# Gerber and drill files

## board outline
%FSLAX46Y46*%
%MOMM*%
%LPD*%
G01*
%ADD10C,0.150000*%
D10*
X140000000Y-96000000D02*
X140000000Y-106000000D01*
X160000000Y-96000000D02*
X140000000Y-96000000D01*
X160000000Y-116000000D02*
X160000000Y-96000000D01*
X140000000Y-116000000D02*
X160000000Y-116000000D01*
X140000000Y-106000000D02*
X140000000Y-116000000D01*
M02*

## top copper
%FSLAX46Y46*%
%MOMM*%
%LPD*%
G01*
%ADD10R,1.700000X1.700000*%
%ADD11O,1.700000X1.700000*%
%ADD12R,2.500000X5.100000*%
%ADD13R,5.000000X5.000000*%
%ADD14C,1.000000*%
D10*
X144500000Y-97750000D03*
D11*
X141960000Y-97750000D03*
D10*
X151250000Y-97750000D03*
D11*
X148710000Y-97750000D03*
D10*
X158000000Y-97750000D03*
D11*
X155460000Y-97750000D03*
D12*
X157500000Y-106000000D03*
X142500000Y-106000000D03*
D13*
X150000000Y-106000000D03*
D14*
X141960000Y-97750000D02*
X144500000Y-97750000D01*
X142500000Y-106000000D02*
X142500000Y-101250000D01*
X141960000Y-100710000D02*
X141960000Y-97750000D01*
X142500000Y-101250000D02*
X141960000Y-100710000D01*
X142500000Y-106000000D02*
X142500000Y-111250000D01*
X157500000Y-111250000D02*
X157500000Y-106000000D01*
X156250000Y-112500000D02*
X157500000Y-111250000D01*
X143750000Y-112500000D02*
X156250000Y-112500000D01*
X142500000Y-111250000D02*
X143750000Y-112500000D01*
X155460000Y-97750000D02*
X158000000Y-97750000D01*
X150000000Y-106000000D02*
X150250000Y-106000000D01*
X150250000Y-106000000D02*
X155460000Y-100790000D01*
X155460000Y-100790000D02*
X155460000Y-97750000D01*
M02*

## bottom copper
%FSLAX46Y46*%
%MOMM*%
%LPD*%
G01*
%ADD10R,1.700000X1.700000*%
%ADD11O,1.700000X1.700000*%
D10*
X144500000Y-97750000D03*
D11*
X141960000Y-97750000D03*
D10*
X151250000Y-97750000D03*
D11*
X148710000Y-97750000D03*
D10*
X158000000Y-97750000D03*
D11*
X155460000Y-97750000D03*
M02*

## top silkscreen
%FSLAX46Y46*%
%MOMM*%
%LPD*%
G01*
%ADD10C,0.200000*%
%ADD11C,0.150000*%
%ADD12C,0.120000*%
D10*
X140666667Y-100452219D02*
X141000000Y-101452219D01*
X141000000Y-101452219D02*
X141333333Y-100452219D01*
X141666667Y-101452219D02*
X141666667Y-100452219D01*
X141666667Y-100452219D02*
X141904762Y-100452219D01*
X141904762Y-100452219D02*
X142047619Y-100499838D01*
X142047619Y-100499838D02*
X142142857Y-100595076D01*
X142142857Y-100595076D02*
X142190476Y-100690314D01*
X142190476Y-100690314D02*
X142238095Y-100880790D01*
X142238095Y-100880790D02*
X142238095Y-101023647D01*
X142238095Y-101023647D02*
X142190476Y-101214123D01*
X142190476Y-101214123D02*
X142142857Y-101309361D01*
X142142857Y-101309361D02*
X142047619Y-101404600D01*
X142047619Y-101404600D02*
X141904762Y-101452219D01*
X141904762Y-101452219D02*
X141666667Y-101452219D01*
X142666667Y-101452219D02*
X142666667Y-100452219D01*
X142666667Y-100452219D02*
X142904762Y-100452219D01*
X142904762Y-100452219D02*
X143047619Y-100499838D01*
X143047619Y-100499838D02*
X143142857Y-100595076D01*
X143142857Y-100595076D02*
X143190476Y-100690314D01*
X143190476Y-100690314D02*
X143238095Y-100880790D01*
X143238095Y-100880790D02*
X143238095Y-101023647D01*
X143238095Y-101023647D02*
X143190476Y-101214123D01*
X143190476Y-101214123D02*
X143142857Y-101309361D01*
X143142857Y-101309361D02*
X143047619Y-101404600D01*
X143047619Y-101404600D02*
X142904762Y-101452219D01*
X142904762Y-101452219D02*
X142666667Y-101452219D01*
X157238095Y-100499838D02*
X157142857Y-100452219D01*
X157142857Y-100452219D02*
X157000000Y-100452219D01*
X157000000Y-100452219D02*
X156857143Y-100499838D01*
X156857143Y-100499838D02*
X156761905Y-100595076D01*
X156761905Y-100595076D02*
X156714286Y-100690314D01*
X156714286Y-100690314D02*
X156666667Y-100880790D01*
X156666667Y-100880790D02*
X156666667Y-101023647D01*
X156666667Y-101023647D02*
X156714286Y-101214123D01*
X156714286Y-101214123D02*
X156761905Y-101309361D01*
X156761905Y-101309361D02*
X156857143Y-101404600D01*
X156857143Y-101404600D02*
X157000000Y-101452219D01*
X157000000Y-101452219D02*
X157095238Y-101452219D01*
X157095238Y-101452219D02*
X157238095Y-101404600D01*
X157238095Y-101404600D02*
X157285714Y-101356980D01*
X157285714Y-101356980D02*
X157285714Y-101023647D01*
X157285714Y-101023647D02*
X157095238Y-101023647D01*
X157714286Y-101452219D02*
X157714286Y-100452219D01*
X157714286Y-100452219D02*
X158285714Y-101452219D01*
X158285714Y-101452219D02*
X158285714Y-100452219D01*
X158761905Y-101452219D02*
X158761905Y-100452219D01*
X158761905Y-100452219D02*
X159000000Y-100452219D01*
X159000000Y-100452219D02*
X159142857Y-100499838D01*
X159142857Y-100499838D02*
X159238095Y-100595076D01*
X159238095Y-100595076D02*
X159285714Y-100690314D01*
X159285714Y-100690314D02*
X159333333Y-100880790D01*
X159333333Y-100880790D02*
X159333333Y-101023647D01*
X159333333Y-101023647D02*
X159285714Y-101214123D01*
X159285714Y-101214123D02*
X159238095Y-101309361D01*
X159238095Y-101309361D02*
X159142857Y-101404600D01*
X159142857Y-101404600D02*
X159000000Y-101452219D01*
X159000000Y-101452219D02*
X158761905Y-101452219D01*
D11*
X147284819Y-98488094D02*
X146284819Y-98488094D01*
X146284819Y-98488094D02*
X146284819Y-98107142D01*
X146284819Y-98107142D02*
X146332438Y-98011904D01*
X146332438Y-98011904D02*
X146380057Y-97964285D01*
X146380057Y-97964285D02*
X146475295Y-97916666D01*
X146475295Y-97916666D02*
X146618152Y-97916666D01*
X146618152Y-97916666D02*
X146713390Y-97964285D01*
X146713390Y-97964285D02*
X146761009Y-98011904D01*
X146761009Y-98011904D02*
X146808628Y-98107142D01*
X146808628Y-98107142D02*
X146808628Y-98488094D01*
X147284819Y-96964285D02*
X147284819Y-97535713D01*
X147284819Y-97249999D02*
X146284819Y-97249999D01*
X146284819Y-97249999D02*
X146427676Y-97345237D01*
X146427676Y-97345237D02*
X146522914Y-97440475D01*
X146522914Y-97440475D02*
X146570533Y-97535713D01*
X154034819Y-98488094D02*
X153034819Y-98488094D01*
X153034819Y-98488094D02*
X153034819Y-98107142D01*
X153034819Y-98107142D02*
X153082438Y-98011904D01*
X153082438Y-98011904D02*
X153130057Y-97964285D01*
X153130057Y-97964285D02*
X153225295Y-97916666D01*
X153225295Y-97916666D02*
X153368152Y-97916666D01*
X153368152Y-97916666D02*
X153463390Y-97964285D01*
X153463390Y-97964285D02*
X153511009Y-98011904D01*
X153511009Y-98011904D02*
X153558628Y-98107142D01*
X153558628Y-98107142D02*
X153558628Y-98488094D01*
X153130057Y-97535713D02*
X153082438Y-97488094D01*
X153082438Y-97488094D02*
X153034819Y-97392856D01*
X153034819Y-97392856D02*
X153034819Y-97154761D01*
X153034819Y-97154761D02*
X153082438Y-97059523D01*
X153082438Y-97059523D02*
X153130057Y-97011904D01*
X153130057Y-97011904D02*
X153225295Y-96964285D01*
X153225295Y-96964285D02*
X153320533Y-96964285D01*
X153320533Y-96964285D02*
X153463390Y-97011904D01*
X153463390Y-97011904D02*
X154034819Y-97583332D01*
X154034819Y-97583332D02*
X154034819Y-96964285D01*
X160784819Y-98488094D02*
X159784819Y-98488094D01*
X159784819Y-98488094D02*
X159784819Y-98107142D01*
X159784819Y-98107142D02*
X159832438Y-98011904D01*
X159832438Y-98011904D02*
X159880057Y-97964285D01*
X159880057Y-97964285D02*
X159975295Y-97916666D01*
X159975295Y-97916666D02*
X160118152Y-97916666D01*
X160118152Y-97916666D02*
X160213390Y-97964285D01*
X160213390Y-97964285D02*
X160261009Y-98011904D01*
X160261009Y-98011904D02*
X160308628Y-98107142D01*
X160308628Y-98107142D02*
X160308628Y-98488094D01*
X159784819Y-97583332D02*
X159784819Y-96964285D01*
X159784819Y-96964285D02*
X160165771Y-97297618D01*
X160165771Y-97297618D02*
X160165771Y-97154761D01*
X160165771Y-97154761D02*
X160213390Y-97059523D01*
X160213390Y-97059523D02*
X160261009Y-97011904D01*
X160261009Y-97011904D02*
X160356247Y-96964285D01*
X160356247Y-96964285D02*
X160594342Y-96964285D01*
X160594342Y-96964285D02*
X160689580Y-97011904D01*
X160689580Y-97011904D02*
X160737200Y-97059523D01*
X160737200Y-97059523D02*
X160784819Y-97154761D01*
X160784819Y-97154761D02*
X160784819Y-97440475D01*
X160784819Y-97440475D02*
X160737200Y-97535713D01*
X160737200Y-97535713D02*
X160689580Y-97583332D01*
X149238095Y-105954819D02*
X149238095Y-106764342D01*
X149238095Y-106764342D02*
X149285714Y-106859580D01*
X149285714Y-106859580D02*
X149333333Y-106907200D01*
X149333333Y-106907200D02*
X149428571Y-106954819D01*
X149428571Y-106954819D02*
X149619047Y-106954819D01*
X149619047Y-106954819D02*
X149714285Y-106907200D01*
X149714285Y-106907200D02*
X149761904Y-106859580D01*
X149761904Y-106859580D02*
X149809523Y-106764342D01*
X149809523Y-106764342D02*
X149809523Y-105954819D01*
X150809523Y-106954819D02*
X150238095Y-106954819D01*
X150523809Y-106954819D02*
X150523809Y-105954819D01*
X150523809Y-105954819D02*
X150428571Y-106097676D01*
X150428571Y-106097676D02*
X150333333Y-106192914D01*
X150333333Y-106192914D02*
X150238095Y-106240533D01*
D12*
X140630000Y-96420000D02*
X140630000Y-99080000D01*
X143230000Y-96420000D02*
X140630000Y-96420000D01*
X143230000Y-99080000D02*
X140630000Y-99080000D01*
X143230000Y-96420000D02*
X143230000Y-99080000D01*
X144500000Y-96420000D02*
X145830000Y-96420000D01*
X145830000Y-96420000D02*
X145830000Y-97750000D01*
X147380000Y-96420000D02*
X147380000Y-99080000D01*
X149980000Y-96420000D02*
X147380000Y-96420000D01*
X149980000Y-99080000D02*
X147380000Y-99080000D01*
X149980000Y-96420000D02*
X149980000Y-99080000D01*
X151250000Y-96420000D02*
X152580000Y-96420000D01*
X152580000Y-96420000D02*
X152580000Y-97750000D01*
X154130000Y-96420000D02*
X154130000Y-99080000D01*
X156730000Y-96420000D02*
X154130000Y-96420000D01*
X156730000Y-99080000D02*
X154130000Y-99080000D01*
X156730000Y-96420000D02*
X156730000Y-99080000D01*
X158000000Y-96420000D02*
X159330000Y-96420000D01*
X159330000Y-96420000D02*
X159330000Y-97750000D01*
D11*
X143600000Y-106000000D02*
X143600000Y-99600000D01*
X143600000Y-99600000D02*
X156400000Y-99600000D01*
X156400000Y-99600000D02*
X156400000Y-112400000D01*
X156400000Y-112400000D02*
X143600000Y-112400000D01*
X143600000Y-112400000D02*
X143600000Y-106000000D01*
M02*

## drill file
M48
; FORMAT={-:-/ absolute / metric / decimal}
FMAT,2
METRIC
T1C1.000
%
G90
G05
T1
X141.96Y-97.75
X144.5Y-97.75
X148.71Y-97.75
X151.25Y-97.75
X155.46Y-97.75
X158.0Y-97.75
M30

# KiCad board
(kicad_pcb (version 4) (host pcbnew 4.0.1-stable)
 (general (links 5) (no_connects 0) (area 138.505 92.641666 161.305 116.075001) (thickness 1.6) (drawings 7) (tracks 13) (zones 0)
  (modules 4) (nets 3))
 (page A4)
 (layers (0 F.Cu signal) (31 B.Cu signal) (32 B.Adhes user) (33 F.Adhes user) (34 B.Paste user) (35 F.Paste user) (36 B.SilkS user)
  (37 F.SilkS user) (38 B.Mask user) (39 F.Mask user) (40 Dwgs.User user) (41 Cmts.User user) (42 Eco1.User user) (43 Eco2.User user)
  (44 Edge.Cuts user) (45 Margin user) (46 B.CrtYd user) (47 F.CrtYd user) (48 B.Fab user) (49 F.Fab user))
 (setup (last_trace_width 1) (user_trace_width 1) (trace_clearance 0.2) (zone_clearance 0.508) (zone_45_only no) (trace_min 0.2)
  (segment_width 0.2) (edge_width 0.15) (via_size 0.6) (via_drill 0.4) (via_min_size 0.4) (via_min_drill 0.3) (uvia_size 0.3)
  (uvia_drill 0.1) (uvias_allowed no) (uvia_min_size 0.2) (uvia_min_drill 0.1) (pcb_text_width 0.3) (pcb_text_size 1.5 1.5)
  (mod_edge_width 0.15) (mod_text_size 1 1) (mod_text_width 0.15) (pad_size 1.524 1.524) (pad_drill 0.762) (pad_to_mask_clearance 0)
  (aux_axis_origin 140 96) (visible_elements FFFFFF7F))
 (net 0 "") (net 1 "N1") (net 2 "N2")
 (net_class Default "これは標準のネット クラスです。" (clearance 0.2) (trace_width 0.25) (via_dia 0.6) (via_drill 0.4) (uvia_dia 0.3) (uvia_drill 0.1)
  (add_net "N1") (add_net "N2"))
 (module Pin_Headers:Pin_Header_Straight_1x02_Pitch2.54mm (layer F.Cu) (at 144.5 97.75 270)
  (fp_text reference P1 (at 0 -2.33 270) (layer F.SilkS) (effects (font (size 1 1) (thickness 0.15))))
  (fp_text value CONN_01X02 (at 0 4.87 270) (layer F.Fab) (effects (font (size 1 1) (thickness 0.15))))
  (fp_line (start -1.33 3.87) (end 1.33 3.87) (layer F.SilkS) (width 0.12))
  (fp_line (start -1.33 1.27) (end -1.33 3.87) (layer F.SilkS) (width 0.12))
  (fp_line (start 1.33 1.27) (end 1.33 3.87) (layer F.SilkS) (width 0.12))
  (fp_line (start -1.33 1.27) (end 1.33 1.27) (layer F.SilkS) (width 0.12))
  (fp_line (start -1.33 0) (end -1.33 -1.33) (layer F.SilkS) (width 0.12))
  (fp_line (start -1.33 -1.33) (end 0 -1.33) (layer F.SilkS) (width 0.12))
  (pad 1 thru_hole rect (at 0 0 270) (size 1.7 1.7) (drill 1) (layers *.Cu *.Mask) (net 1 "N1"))
  (pad 2 thru_hole oval (at 0 2.54 270) (size 1.7 1.7) (drill 1) (layers *.Cu *.Mask) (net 1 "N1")))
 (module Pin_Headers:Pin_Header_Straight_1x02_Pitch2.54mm (layer F.Cu) (at 151.25 97.75 270)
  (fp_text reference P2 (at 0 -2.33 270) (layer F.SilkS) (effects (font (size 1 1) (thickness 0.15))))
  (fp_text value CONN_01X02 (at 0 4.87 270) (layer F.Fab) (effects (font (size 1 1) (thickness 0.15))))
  (fp_line (start -1.33 3.87) (end 1.33 3.87) (layer F.SilkS) (width 0.12))
  (fp_line (start -1.33 1.27) (end -1.33 3.87) (layer F.SilkS) (width 0.12))
  (fp_line (start 1.33 1.27) (end 1.33 3.87) (layer F.SilkS) (width 0.12))
  (fp_line (start -1.33 1.27) (end 1.33 1.27) (layer F.SilkS) (width 0.12))
  (fp_line (start -1.33 0) (end -1.33 -1.33) (layer F.SilkS) (width 0.12))
  (fp_line (start -1.33 -1.33) (end 0 -1.33) (layer F.SilkS) (width 0.12))
  (pad 1 thru_hole rect (at 0 0 270) (size 1.7 1.7) (drill 1) (layers *.Cu *.Mask))
  (pad 2 thru_hole oval (at 0 2.54 270) (size 1.7 1.7) (drill 1) (layers *.Cu *.Mask)))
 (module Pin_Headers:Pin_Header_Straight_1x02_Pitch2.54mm (layer F.Cu) (at 158 97.75 270)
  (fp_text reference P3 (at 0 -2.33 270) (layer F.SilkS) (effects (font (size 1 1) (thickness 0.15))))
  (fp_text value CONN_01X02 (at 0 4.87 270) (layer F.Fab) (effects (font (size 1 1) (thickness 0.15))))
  (fp_line (start -1.33 3.87) (end 1.33 3.87) (layer F.SilkS) (width 0.12))
  (fp_line (start -1.33 1.27) (end -1.33 3.87) (layer F.SilkS) (width 0.12))
  (fp_line (start 1.33 1.27) (end 1.33 3.87) (layer F.SilkS) (width 0.12))
  (fp_line (start -1.33 1.27) (end 1.33 1.27) (layer F.SilkS) (width 0.12))
  (fp_line (start -1.33 0) (end -1.33 -1.33) (layer F.SilkS) (width 0.12))
  (fp_line (start -1.33 -1.33) (end 0 -1.33) (layer F.SilkS) (width 0.12))
  (pad 1 thru_hole rect (at 0 0 270) (size 1.7 1.7) (drill 1) (layers *.Cu *.Mask) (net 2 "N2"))
  (pad 2 thru_hole oval (at 0 2.54 270) (size 1.7 1.7) (drill 1) (layers *.Cu *.Mask) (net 2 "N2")))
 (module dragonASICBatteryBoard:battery (layer F.Cu) (at 150 106)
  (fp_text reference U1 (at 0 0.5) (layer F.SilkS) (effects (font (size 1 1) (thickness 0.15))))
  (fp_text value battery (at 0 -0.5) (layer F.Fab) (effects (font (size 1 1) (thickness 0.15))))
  (fp_line (start -6.4 0) (end -6.4 -6.4) (layer F.SilkS) (width 0.15))
  (fp_line (start -6.4 -6.4) (end 6.4 -6.4) (layer F.SilkS) (width 0.15))
  (fp_line (start 6.4 -6.4) (end 6.4 6.4) (layer F.SilkS) (width 0.15))
  (fp_line (start 6.4 6.4) (end -6.4 6.4) (layer F.SilkS) (width 0.15))
  (fp_line (start -6.4 6.4) (end -6.4 0) (layer F.SilkS) (width 0.15))
  (pad 2 smd rect (at 7.5 0) (size 2.5 5.1) (layers F.Cu F.Paste F.Mask) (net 1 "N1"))
  (pad 2 smd rect (at -7.5 0) (size 2.5 5.1) (layers F.Cu F.Paste F.Mask) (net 1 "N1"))
  (pad 1 smd rect (at 0 0) (size 5 5) (layers F.Cu F.Paste F.Mask) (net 2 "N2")))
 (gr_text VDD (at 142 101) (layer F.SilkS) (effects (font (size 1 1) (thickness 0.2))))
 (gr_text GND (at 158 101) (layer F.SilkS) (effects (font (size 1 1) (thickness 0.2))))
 (gr_line (start 140 96) (end 140 106) (angle 90) (layer Edge.Cuts) (width 0.15))
 (gr_line (start 160 96) (end 140 96) (angle 90) (layer Edge.Cuts) (width 0.15))
 (gr_line (start 160 116) (end 160 96) (angle 90) (layer Edge.Cuts) (width 0.15))
 (gr_line (start 140 116) (end 160 116) (angle 90) (layer Edge.Cuts) (width 0.15))
 (gr_line (start 140 106) (end 140 116) (angle 90) (layer Edge.Cuts) (width 0.15))
 (segment (start 141.96 97.75) (end 144.5 97.75) (width 1) (layer F.Cu) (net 1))
 (segment (start 142.5 106) (end 142.5 101.25) (width 1) (layer F.Cu) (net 1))
 (segment (start 141.96 100.71) (end 141.96 97.75) (width 1) (layer F.Cu) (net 1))
 (segment (start 142.5 101.25) (end 141.96 100.71) (width 1) (layer F.Cu) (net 1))
 (segment (start 142.5 106) (end 142.5 111.25) (width 1) (layer F.Cu) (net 1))
 (segment (start 157.5 111.25) (end 157.5 106) (width 1) (layer F.Cu) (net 1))
 (segment (start 156.25 112.5) (end 157.5 111.25) (width 1) (layer F.Cu) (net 1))
 (segment (start 143.75 112.5) (end 156.25 112.5) (width 1) (layer F.Cu) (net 1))
 (segment (start 142.5 111.25) (end 143.75 112.5) (width 1) (layer F.Cu) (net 1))
 (segment (start 155.46 97.75) (end 158 97.75) (width 1) (layer F.Cu) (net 2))
 (segment (start 150 106) (end 150.25 106) (width 1) (layer F.Cu) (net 2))
 (segment (start 150.25 106) (end 155.46 100.79) (width 1) (layer F.Cu) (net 2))
 (segment (start 155.46 100.79) (end 155.46 97.75) (width 1) (layer F.Cu) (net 2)))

